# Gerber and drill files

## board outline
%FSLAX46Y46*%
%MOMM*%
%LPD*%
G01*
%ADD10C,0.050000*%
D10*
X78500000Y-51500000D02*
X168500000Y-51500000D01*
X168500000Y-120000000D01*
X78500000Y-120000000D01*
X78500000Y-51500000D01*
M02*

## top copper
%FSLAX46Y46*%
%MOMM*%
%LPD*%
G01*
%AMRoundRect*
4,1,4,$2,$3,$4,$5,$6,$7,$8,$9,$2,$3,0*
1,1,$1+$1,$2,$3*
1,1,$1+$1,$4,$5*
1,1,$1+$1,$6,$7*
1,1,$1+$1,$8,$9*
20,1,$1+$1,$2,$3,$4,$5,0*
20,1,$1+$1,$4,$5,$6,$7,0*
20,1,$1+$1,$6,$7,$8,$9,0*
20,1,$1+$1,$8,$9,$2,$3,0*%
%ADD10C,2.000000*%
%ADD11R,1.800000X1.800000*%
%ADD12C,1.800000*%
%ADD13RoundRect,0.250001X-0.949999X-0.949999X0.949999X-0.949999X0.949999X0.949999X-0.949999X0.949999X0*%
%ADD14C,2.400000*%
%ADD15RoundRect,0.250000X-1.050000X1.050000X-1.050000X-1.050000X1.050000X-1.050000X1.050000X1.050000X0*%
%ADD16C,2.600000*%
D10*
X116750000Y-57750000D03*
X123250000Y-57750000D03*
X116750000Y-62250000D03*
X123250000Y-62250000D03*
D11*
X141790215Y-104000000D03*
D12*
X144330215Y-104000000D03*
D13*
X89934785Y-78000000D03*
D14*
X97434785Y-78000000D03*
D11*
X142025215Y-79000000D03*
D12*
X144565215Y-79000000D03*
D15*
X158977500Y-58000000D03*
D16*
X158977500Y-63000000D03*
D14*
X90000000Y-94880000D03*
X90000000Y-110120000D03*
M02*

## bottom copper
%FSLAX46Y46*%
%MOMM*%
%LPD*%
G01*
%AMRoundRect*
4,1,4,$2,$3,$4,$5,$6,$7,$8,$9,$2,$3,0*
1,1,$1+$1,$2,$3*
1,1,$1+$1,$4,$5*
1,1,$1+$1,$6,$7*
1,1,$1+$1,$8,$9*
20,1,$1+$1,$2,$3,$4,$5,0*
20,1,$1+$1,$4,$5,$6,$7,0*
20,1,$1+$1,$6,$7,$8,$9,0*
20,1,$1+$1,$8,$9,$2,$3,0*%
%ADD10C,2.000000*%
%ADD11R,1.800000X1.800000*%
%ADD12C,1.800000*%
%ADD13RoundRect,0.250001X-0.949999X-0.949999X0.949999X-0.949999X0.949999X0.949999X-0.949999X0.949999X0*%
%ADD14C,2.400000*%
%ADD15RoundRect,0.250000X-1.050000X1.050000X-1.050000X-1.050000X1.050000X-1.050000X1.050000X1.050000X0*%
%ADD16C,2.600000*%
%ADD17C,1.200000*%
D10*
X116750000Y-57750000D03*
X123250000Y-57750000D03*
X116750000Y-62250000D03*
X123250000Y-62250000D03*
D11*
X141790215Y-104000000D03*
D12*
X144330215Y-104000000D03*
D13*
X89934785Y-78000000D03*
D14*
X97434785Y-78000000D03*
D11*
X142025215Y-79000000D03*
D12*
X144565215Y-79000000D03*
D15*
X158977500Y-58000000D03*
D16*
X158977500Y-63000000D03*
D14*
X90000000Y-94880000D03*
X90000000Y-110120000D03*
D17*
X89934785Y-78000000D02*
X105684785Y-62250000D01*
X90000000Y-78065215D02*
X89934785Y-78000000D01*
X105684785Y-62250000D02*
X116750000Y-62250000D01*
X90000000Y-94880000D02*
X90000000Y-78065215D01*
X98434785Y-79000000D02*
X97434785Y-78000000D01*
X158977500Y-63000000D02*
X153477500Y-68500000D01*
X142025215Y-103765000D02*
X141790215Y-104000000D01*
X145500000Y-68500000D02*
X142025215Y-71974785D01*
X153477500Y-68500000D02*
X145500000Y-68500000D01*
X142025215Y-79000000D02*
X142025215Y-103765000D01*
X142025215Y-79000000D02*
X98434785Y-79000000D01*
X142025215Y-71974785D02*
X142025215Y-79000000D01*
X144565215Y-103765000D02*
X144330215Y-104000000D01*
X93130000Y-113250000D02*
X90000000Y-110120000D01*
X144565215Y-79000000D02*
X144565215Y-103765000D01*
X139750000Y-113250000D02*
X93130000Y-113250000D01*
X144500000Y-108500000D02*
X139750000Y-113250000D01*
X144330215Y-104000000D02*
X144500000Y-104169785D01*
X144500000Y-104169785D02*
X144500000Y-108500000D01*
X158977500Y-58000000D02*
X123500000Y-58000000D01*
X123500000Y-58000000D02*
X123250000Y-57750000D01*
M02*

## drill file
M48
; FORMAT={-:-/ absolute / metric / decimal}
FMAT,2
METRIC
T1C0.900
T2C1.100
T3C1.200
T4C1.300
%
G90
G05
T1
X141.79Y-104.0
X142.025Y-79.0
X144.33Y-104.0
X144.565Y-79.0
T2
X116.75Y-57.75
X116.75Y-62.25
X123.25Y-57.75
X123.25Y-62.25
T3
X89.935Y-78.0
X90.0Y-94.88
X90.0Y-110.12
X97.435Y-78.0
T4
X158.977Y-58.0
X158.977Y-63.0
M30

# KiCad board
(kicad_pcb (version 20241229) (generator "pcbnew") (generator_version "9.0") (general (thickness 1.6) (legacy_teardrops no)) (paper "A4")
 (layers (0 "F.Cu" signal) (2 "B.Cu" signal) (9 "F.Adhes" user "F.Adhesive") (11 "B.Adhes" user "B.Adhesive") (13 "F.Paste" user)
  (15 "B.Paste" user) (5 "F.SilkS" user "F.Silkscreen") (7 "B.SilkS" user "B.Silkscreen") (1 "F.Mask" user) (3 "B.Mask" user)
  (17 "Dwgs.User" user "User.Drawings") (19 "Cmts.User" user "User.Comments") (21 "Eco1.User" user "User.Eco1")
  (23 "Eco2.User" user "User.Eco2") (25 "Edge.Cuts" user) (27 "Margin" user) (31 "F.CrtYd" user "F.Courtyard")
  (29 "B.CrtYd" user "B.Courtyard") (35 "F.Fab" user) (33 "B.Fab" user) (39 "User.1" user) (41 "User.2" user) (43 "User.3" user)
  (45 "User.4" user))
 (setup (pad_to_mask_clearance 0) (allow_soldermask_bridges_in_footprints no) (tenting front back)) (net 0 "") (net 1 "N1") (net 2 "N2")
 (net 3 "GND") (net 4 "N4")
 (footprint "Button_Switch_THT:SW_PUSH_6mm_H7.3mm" (layer "F.Cu") (at 116.75 57.75)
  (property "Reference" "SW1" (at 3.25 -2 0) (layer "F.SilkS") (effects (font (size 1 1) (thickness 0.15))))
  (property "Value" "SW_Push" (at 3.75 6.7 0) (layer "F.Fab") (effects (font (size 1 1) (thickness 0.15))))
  (pad "1" thru_hole circle (at 0 0 90) (size 2 2) (drill 1.1) (layers "*.Cu" "*.Mask") (remove_unused_layers no) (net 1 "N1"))
  (pad "1" thru_hole circle (at 6.5 0 90) (size 2 2) (drill 1.1) (layers "*.Cu" "*.Mask") (remove_unused_layers no) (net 1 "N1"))
  (pad "2" thru_hole circle (at 0 4.5 90) (size 2 2) (drill 1.1) (layers "*.Cu" "*.Mask") (remove_unused_layers no) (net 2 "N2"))
  (pad "2" thru_hole circle (at 6.5 4.5 90) (size 2 2) (drill 1.1) (layers "*.Cu" "*.Mask") (remove_unused_layers no) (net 2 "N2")))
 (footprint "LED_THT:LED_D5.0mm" (layer "F.Cu") (at 141.790215 104)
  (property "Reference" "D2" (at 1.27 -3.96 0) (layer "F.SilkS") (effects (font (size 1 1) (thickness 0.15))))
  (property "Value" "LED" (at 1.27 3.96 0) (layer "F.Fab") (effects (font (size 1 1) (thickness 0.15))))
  (pad "1" thru_hole rect (at 0 0) (size 1.8 1.8) (drill 0.9) (layers "*.Cu" "*.Mask") (remove_unused_layers no) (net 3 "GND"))
  (pad "2" thru_hole circle (at 2.54 0) (size 1.8 1.8) (drill 0.9) (layers "*.Cu" "*.Mask") (remove_unused_layers no) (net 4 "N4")))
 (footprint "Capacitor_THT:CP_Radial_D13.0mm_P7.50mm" (layer "F.Cu") (at 89.934785 78)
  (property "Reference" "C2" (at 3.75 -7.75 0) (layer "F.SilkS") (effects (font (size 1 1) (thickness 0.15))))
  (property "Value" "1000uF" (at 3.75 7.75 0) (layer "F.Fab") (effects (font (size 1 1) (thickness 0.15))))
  (pad "1" thru_hole roundrect (at 0 0) (size 2.4 2.4) (drill 1.2) (layers "*.Cu" "*.Mask") (remove_unused_layers no)
   (roundrect_rratio 0.104167) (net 2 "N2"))
  (pad "2" thru_hole circle (at 7.5 0) (size 2.4 2.4) (drill 1.2) (layers "*.Cu" "*.Mask") (remove_unused_layers no) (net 3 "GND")))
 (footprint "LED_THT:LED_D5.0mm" (layer "F.Cu") (at 142.025215 79)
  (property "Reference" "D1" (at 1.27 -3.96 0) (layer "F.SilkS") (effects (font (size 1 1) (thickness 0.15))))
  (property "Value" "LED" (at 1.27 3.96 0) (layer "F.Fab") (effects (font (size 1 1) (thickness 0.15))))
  (pad "1" thru_hole rect (at 0 0) (size 1.8 1.8) (drill 0.9) (layers "*.Cu" "*.Mask") (remove_unused_layers no) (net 3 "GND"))
  (pad "2" thru_hole circle (at 2.54 0) (size 1.8 1.8) (drill 0.9) (layers "*.Cu" "*.Mask") (remove_unused_layers no) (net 4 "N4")))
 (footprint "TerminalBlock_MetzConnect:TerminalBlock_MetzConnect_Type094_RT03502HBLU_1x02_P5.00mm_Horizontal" (layer "F.Cu")
  (at 158.9775 58 -90)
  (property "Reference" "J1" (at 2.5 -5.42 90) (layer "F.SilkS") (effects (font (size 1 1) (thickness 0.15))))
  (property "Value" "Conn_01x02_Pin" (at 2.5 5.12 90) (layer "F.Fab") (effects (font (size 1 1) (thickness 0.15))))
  (pad "1" thru_hole roundrect (at 0 0 270) (size 2.6 2.6) (drill 1.3) (layers "*.Cu" "*.Mask") (remove_unused_layers no)
   (roundrect_rratio 0.096154) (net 1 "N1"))
  (pad "2" thru_hole circle (at 5 0 270) (size 2.6 2.6) (drill 1.3) (layers "*.Cu" "*.Mask") (remove_unused_layers no) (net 3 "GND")))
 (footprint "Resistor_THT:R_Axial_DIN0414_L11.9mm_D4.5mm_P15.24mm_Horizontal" (layer "F.Cu") (at 90 94.88 -90)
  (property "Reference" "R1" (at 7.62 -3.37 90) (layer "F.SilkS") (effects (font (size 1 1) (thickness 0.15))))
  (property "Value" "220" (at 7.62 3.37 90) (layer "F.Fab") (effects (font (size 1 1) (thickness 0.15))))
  (pad "1" thru_hole circle (at 0 0 270) (size 2.4 2.4) (drill 1.2) (layers "*.Cu" "*.Mask") (remove_unused_layers no) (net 2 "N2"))
  (pad "2" thru_hole circle (at 15.24 0 270) (size 2.4 2.4) (drill 1.2) (layers "*.Cu" "*.Mask") (remove_unused_layers no) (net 4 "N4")))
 (gr_rect (start 78.5 51.5) (end 168.5 120) (stroke (width 0.05) (type default)) (fill no) (layer "Edge.Cuts"))
 (segment (start 89.934785 78) (end 105.684785 62.25) (width 1.2) (layer "B.Cu") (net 2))
 (segment (start 90 78.065215) (end 89.934785 78) (width 1.2) (layer "B.Cu") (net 2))
 (segment (start 105.684785 62.25) (end 116.75 62.25) (width 1.2) (layer "B.Cu") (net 2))
 (segment (start 90 94.88) (end 90 78.065215) (width 1.2) (layer "B.Cu") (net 2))
 (segment (start 98.434785 79) (end 97.434785 78) (width 1.2) (layer "B.Cu") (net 3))
 (segment (start 158.9775 63) (end 153.4775 68.5) (width 1.2) (layer "B.Cu") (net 3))
 (segment (start 142.025215 103.765) (end 141.790215 104) (width 1.2) (layer "B.Cu") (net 3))
 (segment (start 145.5 68.5) (end 142.025215 71.974785) (width 1.2) (layer "B.Cu") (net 3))
 (segment (start 153.4775 68.5) (end 145.5 68.5) (width 1.2) (layer "B.Cu") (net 3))
 (segment (start 142.025215 79) (end 142.025215 103.765) (width 1.2) (layer "B.Cu") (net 3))
 (segment (start 142.025215 79) (end 98.434785 79) (width 1.2) (layer "B.Cu") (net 3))
 (segment (start 142.025215 71.974785) (end 142.025215 79) (width 1.2) (layer "B.Cu") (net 3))
 (segment (start 144.565215 103.765) (end 144.330215 104) (width 1.2) (layer "B.Cu") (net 4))
 (segment (start 93.13 113.25) (end 90 110.12) (width 1.2) (layer "B.Cu") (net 4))
 (segment (start 144.565215 79) (end 144.565215 103.765) (width 1.2) (layer "B.Cu") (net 4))
 (segment (start 139.75 113.25) (end 93.13 113.25) (width 1.2) (layer "B.Cu") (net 4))
 (segment (start 144.5 108.5) (end 139.75 113.25) (width 1.2) (layer "B.Cu") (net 4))
 (segment (start 144.330215 104) (end 144.5 104.169785) (width 1.2) (layer "B.Cu") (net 4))
 (segment (start 144.5 104.169785) (end 144.5 108.5) (width 1.2) (layer "B.Cu") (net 4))
 (segment (start 158.9775 58) (end 123.5 58) (width 1.2) (layer "B.Cu") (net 1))
 (segment (start 123.5 58) (end 123.25 57.75) (width 1.2) (layer "B.Cu") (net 1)))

